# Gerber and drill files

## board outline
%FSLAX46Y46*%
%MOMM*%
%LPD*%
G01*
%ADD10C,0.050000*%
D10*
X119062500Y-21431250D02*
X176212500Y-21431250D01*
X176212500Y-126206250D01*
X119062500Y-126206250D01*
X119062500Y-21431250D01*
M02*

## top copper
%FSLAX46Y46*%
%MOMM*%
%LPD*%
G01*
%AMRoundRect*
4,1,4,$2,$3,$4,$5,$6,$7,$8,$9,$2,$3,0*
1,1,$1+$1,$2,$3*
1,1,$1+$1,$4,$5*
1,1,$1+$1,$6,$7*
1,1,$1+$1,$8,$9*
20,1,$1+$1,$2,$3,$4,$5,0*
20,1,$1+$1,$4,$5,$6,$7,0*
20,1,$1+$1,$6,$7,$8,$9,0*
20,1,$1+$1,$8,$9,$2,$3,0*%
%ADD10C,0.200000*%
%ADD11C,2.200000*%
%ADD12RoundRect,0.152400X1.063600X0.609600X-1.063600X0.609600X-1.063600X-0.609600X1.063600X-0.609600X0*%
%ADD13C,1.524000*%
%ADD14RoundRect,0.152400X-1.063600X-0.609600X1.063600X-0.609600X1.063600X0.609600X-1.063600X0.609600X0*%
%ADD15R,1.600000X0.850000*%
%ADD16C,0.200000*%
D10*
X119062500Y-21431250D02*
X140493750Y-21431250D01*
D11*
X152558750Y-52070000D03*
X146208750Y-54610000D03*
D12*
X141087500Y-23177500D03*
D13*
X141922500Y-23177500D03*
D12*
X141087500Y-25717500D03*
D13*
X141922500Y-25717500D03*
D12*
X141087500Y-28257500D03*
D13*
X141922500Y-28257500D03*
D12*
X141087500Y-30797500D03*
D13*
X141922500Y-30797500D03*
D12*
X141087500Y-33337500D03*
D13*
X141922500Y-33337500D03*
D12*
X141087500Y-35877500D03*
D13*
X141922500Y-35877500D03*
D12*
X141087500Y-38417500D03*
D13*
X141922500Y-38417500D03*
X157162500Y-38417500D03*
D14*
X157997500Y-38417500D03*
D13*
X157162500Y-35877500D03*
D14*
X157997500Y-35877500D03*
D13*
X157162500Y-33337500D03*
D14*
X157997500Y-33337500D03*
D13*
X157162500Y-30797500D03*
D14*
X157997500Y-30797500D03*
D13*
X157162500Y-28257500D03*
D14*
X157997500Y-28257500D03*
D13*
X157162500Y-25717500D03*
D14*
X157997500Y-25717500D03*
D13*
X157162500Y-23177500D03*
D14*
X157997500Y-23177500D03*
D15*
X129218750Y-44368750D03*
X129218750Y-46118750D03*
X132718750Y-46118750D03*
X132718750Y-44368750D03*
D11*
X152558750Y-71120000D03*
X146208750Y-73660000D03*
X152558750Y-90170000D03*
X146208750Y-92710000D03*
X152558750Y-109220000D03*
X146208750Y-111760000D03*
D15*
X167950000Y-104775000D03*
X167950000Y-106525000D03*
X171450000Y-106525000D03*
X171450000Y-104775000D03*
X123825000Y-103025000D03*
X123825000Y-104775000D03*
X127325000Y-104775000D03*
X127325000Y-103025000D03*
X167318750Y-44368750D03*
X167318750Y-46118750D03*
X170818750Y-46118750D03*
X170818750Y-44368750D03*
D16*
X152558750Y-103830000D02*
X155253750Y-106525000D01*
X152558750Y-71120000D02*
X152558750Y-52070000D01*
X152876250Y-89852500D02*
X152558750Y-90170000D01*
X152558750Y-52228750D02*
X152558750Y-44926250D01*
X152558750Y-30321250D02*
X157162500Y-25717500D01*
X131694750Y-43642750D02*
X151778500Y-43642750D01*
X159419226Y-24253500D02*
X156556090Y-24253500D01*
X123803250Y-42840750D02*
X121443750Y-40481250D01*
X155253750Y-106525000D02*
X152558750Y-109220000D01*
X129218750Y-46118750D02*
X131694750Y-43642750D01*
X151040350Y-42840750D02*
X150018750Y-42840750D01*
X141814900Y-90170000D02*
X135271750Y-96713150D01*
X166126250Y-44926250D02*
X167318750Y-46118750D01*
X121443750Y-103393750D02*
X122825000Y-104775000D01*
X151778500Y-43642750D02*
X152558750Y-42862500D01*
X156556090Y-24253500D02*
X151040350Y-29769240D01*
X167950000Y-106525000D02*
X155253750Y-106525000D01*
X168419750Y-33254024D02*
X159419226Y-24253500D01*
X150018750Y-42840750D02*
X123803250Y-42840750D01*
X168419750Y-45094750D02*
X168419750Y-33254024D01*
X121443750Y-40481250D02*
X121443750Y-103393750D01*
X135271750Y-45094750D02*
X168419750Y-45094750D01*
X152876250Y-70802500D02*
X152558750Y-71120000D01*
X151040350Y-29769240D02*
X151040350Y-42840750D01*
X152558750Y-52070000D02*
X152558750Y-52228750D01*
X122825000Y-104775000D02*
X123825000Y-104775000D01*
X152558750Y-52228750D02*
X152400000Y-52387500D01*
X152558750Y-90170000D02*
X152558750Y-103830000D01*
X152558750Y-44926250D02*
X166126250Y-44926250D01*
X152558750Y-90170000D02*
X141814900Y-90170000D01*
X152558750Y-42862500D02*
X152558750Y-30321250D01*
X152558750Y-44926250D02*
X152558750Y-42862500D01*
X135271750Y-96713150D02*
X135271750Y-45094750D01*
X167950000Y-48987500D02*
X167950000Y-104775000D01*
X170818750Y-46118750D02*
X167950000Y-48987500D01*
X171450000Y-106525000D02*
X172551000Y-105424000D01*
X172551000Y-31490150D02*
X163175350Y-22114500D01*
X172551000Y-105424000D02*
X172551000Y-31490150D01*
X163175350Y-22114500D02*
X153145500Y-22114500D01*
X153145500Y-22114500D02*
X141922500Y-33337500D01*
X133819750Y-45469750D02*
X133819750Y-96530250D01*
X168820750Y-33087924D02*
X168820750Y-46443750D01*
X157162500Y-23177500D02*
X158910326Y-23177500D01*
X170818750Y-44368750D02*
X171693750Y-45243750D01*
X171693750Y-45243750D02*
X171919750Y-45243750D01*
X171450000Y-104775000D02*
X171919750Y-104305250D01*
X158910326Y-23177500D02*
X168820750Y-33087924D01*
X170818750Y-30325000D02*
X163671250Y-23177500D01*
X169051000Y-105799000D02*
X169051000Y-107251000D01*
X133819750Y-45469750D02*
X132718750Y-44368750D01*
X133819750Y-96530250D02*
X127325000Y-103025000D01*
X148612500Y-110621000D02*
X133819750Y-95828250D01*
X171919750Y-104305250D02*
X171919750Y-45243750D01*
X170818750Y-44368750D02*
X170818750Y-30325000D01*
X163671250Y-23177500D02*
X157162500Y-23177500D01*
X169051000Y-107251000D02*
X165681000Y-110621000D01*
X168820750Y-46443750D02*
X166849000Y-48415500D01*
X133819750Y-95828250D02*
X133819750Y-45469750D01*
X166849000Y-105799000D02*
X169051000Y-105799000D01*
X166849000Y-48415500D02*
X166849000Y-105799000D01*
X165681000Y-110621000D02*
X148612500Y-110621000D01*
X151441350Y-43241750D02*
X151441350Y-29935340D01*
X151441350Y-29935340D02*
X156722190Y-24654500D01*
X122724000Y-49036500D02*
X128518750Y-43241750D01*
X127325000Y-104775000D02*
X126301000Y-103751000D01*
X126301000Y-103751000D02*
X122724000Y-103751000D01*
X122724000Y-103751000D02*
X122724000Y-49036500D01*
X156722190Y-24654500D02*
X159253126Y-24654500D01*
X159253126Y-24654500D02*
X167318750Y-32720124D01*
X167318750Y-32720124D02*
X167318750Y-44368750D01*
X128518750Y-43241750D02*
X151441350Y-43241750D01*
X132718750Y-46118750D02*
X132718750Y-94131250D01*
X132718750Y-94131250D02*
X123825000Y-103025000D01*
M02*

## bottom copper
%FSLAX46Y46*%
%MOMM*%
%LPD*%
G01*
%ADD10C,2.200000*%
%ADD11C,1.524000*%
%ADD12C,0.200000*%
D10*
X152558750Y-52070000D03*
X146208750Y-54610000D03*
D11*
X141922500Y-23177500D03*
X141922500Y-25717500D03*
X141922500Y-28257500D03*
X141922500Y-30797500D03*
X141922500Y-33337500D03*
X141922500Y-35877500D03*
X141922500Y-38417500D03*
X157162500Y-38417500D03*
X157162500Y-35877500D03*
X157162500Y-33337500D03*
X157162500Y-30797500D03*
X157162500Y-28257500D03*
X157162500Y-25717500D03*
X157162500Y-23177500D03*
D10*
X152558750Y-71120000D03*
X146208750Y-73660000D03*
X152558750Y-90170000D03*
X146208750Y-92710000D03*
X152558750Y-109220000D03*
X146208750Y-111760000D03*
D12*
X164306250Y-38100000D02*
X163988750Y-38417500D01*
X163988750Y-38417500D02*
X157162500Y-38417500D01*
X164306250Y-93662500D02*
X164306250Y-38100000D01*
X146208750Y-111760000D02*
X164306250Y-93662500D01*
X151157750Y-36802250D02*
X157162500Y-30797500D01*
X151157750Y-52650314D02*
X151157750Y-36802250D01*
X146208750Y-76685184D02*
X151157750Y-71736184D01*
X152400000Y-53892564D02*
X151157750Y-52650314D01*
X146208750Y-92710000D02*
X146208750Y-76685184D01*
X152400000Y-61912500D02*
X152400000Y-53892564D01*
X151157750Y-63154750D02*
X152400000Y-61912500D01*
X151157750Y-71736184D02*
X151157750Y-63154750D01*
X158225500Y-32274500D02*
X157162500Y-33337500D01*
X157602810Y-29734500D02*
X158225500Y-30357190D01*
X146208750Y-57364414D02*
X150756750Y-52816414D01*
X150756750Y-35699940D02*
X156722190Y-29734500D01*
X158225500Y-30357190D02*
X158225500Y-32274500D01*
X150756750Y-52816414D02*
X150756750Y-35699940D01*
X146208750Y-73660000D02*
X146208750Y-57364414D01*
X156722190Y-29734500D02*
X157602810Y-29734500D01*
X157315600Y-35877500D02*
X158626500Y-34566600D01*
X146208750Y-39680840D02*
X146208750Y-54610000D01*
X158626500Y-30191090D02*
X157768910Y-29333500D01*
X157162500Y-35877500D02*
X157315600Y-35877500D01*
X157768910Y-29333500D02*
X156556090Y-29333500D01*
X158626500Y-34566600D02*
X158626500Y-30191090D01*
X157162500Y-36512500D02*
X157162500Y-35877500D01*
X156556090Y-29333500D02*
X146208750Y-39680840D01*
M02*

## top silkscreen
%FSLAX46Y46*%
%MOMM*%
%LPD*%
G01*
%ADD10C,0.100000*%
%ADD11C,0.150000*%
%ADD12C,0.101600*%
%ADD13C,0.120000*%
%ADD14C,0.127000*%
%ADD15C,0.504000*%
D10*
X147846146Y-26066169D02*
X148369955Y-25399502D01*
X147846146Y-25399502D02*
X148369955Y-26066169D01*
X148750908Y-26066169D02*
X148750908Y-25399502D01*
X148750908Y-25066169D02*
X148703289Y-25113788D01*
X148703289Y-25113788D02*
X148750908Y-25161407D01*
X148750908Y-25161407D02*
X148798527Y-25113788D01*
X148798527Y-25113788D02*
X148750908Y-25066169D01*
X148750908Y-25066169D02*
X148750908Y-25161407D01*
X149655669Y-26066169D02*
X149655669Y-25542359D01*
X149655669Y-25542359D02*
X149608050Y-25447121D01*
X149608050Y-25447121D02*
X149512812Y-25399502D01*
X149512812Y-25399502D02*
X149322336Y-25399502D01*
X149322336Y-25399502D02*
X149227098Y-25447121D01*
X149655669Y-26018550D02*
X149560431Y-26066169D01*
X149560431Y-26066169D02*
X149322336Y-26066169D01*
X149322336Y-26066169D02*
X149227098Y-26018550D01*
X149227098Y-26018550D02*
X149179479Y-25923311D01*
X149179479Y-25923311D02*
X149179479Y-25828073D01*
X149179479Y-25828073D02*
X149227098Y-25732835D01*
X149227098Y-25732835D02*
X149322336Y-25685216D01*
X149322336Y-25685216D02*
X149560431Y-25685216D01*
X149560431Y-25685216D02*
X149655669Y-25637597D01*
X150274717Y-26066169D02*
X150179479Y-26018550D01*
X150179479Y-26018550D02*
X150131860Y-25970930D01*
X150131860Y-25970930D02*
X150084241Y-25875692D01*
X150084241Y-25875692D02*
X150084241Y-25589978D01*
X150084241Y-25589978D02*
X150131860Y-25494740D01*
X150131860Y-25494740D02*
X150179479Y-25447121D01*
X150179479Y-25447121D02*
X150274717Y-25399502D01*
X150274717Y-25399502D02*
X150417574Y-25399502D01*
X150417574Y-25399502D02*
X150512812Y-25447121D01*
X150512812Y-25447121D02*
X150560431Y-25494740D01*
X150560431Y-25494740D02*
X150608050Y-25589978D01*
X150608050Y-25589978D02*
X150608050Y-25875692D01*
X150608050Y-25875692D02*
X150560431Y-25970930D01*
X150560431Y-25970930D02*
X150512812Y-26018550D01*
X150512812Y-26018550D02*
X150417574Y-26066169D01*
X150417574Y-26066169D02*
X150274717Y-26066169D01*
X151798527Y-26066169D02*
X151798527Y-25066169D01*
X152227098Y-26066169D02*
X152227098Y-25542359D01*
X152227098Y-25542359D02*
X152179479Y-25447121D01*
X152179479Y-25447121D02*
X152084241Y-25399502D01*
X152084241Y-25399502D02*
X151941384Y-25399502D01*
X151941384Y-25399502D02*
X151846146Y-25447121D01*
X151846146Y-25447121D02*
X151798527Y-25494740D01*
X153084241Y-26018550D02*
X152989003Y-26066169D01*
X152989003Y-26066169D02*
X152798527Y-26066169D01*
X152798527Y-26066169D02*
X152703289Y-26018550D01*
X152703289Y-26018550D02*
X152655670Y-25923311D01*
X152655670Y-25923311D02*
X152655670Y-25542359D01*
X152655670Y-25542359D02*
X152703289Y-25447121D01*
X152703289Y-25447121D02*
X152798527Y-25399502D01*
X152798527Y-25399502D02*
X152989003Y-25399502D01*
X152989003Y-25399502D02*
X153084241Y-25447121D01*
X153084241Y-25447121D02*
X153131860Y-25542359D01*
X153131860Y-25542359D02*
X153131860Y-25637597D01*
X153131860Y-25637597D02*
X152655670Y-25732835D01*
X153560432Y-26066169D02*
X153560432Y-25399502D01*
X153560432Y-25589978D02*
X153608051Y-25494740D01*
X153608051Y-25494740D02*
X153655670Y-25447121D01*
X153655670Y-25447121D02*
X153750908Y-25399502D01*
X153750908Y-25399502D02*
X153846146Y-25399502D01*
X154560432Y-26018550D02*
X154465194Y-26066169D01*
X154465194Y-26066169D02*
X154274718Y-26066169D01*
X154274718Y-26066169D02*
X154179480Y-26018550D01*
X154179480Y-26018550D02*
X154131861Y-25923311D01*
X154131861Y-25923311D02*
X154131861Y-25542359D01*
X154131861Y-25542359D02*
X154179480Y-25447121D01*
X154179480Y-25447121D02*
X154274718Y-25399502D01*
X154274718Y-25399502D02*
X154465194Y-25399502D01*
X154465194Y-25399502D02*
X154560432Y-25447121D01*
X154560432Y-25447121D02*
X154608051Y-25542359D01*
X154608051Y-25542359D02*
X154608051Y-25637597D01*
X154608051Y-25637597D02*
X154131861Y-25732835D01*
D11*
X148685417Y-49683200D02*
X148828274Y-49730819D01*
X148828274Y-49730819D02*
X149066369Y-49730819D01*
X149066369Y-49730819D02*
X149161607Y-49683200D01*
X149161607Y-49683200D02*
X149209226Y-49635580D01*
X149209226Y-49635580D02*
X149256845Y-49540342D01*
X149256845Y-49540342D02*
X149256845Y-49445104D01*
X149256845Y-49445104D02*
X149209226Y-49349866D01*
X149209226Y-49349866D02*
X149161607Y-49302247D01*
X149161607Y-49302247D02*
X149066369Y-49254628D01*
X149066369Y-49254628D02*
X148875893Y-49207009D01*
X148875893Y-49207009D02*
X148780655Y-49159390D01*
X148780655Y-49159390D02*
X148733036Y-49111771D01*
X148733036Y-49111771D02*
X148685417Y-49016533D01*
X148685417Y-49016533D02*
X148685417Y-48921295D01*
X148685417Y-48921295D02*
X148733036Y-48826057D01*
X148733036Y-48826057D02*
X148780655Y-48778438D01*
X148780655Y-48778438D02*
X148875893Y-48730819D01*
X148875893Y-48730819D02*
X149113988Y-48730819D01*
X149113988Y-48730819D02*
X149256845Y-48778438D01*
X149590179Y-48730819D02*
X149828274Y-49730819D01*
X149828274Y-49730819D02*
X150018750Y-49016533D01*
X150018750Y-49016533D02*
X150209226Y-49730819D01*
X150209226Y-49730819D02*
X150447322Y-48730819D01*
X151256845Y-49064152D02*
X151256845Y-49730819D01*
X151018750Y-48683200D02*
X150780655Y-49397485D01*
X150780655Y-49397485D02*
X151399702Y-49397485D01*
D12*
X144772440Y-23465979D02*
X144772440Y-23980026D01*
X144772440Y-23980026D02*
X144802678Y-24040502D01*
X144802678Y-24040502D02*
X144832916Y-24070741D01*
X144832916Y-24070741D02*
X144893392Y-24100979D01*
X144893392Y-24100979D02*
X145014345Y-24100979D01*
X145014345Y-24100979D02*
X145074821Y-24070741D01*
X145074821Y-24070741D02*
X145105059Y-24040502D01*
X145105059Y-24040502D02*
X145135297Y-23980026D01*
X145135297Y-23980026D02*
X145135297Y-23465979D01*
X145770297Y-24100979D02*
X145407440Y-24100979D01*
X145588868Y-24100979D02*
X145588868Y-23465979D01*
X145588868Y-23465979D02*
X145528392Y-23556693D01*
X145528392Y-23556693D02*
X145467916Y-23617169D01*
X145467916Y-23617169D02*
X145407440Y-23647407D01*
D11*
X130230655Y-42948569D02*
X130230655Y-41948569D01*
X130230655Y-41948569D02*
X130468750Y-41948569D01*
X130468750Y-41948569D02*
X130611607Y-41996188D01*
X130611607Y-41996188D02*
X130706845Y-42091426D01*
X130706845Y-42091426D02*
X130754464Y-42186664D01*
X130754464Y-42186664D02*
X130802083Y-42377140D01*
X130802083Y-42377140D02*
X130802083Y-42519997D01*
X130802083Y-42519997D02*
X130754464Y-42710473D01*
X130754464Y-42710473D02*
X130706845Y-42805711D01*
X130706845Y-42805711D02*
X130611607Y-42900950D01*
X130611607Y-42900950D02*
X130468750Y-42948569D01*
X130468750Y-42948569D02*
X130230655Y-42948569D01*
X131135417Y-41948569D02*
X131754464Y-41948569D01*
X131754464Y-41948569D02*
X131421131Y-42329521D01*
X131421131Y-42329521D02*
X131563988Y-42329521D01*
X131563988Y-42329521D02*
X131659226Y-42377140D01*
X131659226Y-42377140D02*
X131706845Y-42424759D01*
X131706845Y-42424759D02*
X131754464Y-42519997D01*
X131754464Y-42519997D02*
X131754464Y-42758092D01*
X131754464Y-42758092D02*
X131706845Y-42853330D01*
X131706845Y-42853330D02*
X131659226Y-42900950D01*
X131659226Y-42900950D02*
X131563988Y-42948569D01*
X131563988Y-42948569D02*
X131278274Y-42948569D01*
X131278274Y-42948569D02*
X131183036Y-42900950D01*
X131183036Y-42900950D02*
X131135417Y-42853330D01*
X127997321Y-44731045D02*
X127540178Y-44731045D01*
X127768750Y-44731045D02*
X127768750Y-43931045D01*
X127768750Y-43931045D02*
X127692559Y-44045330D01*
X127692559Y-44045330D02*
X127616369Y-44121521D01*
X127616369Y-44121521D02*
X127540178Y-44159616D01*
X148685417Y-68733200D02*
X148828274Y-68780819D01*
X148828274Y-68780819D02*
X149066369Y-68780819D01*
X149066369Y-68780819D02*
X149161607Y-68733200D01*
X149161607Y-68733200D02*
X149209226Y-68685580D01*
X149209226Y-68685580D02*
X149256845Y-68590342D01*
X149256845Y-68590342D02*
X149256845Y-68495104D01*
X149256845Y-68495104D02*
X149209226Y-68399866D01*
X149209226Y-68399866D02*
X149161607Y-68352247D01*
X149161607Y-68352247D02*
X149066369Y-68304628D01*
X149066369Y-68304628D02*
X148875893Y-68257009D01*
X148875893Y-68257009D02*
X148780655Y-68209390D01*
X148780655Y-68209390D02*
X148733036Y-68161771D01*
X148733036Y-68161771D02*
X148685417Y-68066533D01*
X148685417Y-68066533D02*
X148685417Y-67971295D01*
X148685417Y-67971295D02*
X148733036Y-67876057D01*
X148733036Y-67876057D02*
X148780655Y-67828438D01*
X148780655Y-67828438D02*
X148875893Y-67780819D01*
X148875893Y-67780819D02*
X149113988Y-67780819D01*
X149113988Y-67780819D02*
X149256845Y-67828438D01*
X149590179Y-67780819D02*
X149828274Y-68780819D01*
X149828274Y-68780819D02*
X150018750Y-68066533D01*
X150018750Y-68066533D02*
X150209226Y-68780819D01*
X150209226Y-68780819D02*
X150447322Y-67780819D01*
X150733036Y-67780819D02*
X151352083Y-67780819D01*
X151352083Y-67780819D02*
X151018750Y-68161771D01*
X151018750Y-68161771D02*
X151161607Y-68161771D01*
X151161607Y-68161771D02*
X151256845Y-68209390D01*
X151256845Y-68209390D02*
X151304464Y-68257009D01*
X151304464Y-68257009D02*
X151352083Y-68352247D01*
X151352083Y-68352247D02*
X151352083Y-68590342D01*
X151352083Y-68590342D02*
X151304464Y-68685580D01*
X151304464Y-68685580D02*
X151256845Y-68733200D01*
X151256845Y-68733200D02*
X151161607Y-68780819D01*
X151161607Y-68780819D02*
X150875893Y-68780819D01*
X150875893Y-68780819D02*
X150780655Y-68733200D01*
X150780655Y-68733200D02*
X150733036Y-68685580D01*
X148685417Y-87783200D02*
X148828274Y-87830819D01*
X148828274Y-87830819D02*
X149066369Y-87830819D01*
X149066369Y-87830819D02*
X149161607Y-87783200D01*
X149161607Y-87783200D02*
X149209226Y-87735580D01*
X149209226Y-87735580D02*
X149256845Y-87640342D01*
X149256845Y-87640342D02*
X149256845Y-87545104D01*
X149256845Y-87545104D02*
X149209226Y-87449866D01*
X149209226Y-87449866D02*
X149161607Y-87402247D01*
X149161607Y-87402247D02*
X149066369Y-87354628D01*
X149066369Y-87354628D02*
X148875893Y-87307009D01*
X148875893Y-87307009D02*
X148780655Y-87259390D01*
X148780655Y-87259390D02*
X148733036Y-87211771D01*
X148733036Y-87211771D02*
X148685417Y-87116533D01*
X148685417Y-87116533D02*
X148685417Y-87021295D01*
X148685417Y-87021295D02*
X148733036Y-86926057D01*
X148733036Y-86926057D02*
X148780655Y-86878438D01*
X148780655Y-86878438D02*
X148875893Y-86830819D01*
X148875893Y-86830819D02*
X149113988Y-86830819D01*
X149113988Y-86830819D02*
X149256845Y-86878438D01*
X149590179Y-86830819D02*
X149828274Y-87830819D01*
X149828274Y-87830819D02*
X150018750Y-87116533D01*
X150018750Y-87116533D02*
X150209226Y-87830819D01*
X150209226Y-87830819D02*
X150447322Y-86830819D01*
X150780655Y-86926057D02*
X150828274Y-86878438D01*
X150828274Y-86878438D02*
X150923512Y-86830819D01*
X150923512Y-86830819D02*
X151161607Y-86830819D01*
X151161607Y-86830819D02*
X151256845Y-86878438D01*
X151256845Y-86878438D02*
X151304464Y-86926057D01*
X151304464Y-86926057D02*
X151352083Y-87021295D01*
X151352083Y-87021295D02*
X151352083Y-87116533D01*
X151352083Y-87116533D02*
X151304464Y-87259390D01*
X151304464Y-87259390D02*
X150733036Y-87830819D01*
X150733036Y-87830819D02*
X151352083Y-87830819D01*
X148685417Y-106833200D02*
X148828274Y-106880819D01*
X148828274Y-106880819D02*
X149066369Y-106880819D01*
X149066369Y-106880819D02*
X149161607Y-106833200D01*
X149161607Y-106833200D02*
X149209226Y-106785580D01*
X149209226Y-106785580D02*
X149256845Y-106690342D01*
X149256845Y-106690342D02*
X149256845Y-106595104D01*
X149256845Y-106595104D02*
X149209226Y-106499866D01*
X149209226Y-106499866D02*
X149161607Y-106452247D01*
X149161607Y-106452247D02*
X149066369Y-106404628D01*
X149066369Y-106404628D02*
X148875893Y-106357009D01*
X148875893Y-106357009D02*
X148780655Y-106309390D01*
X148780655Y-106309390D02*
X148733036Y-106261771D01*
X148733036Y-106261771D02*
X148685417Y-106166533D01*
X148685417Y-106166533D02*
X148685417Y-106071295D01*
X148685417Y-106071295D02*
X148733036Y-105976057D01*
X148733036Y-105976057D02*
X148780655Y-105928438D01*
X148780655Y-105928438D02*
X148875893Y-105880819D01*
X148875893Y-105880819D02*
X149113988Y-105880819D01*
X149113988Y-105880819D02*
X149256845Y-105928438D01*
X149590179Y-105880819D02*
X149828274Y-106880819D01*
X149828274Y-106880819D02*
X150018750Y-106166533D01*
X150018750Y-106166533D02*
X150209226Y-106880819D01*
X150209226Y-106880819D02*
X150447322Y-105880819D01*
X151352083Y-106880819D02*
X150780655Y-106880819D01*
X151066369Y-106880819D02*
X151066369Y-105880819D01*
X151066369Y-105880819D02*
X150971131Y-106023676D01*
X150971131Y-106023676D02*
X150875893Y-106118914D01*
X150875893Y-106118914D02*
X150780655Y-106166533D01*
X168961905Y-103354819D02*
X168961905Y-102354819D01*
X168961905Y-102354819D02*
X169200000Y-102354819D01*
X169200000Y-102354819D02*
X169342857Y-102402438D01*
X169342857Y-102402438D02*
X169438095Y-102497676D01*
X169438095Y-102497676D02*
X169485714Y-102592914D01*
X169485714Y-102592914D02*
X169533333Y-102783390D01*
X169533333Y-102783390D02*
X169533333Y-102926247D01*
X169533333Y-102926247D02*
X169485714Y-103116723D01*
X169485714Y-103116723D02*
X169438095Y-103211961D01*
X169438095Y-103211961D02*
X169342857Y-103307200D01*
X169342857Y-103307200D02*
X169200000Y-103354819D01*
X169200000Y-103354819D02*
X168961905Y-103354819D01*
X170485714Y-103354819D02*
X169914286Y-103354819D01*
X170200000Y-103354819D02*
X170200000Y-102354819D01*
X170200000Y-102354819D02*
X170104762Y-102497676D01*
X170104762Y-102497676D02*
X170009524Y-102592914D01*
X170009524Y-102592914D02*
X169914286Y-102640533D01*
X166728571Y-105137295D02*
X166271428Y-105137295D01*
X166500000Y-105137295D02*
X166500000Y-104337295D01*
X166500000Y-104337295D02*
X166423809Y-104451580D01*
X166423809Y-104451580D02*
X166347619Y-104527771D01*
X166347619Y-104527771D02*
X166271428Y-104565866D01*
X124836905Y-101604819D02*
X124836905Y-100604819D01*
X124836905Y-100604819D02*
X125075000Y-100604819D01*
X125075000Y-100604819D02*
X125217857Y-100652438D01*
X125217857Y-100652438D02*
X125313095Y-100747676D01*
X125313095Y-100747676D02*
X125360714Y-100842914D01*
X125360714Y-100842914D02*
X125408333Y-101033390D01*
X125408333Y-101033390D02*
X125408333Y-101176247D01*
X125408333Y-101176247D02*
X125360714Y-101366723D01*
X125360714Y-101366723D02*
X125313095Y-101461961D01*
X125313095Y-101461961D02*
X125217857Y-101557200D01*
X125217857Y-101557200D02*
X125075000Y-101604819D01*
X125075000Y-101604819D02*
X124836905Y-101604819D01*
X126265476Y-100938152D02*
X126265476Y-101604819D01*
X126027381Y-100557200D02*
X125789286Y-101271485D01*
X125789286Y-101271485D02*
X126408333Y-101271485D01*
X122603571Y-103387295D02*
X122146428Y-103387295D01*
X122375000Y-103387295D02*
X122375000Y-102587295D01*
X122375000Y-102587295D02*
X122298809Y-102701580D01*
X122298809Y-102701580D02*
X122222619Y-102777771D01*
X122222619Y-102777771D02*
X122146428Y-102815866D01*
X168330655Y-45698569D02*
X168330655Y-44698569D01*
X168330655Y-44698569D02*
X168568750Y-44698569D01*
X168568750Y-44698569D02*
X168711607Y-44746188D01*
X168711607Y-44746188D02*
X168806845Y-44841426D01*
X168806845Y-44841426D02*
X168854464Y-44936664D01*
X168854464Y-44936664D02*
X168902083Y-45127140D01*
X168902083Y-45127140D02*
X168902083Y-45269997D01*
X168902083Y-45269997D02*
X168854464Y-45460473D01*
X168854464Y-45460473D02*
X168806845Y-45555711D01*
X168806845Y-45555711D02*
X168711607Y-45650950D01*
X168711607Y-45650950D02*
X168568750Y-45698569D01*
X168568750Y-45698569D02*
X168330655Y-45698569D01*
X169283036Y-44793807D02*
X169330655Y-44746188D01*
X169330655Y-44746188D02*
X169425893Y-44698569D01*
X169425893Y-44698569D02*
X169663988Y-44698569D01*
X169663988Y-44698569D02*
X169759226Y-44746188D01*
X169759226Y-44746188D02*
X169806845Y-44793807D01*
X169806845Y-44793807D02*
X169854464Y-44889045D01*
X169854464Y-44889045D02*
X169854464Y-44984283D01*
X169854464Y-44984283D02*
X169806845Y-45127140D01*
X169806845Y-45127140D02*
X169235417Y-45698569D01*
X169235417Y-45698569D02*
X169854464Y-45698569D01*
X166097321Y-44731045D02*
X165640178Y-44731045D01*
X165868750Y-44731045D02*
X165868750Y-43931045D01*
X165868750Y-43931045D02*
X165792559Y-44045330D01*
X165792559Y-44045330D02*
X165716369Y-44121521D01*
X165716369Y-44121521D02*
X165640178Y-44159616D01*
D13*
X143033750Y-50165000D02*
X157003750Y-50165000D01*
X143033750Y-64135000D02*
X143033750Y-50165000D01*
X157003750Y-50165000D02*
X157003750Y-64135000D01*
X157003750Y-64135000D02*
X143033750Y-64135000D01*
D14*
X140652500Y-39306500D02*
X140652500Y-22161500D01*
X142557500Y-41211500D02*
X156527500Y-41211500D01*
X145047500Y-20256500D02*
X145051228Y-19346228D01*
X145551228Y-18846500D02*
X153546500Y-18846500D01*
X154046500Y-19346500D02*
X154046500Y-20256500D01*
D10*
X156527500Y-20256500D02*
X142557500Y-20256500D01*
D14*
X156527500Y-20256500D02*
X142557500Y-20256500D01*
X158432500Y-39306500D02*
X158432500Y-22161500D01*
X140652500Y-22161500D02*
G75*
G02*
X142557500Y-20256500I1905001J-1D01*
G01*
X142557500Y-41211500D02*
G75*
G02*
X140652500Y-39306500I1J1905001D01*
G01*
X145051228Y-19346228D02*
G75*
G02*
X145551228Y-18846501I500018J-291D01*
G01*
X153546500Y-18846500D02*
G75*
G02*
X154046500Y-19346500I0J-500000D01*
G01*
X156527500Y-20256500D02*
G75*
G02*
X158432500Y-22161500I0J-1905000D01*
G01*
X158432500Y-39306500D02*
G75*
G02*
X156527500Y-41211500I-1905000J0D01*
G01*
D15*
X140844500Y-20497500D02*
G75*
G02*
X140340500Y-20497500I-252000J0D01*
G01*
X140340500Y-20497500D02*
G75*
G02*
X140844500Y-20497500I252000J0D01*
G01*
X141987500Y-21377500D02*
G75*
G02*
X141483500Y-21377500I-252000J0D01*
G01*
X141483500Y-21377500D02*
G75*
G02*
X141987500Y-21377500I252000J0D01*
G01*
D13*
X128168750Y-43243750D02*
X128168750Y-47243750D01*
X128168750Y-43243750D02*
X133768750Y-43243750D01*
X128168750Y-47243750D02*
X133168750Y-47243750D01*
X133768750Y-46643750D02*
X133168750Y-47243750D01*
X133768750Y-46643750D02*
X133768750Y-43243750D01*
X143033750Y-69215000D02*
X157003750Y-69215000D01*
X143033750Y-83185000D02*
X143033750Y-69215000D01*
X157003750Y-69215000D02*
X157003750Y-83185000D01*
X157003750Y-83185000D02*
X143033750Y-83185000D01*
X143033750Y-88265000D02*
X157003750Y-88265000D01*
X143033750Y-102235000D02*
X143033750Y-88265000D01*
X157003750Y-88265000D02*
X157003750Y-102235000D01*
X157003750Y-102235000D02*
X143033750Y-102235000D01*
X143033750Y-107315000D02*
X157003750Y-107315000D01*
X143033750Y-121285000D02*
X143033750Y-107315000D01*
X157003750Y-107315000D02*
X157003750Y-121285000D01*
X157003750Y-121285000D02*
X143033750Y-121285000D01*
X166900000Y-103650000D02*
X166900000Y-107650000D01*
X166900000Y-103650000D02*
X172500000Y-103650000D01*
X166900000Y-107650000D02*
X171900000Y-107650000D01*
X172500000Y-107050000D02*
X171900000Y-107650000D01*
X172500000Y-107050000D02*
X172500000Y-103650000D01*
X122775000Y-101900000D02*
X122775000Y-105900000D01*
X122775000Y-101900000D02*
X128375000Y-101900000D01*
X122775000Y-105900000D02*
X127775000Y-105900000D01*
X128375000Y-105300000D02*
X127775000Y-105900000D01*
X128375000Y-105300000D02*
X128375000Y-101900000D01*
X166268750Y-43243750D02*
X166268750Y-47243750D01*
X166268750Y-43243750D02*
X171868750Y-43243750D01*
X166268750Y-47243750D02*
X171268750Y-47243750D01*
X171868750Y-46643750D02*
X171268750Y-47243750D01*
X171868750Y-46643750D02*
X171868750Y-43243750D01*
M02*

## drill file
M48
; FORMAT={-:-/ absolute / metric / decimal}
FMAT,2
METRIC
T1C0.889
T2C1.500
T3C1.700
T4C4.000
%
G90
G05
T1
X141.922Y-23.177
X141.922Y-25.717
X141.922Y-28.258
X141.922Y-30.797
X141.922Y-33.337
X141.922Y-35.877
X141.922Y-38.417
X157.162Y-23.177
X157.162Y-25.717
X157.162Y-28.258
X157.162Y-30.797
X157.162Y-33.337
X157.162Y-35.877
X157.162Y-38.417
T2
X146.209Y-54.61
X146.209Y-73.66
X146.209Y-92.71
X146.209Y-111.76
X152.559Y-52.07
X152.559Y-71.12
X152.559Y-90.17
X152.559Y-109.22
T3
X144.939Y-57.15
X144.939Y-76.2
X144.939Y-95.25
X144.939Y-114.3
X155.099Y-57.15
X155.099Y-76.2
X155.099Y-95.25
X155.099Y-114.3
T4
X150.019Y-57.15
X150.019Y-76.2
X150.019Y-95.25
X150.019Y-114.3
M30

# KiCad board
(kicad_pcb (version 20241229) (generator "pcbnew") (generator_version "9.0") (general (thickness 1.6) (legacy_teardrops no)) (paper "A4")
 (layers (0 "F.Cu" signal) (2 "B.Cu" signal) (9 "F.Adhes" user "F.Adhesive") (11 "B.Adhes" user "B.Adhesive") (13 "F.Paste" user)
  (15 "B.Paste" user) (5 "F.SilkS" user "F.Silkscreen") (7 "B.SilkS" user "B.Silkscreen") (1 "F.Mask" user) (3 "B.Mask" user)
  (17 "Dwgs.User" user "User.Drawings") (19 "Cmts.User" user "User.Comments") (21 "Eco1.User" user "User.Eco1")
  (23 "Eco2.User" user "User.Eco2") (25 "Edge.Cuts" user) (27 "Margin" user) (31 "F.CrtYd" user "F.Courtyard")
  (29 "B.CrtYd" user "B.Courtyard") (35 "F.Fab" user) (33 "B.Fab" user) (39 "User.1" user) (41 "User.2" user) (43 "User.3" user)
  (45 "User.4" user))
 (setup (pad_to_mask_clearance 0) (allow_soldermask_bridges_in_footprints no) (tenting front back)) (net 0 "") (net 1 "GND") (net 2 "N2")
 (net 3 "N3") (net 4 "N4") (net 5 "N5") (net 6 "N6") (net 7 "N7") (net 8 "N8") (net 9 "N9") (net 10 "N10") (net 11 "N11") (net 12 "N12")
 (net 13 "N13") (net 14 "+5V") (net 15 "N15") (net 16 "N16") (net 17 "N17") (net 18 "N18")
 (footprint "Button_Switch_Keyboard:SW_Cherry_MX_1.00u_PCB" (layer "F.Cu") (at 152.55875 52.07)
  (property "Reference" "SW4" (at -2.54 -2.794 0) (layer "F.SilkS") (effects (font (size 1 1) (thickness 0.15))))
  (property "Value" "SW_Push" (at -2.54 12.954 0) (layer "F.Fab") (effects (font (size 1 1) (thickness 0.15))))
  (fp_line (start -9.525 -1.905) (end 4.445 -1.905) (stroke (width 0.12) (type solid)) (layer "F.SilkS"))
  (fp_line (start -9.525 12.065) (end -9.525 -1.905) (stroke (width 0.12) (type solid)) (layer "F.SilkS"))
  (fp_line (start 4.445 -1.905) (end 4.445 12.065) (stroke (width 0.12) (type solid)) (layer "F.SilkS"))
  (fp_line (start 4.445 12.065) (end -9.525 12.065) (stroke (width 0.12) (type solid)) (layer "F.SilkS"))
  (pad "" np_thru_hole circle (at -7.62 5.08) (size 1.7 1.7) (drill 1.7) (layers "*.Cu" "*.Mask"))
  (pad "" np_thru_hole circle (at -2.54 5.08) (size 4 4) (drill 4) (layers "*.Cu" "*.Mask"))
  (pad "" np_thru_hole circle (at 2.54 5.08) (size 1.7 1.7) (drill 1.7) (layers "*.Cu" "*.Mask"))
  (pad "1" thru_hole circle (at 0 0) (size 2.2 2.2) (drill 1.5) (layers "*.Cu" "*.Mask") (remove_unused_layers no) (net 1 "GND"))
  (pad "2" thru_hole circle (at -6.35 2.54) (size 2.2 2.2) (drill 1.5) (layers "*.Cu" "*.Mask") (remove_unused_layers no) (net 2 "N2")))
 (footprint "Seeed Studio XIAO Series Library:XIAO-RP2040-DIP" (layer "F.Cu") (at 149.5425 30.7975)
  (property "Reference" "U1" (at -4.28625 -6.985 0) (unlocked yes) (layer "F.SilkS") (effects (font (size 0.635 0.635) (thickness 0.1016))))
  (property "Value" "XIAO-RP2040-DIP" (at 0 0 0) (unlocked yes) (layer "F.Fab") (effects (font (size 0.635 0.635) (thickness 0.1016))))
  (fp_line (start -8.89 8.509) (end -8.89 -8.636) (stroke (width 0.127) (type solid)) (layer "F.SilkS"))
  (fp_line (start -6.985 10.414) (end 6.985 10.414) (stroke (width 0.127) (type solid)) (layer "F.SilkS"))
  (fp_line (start -4.495 -10.541) (end -4.491272 -11.451272) (stroke (width 0.127) (type solid)) (layer "F.SilkS"))
  (fp_line (start -3.991272 -11.951) (end 4.004 -11.951) (stroke (width 0.127) (type solid)) (layer "F.SilkS"))
  (fp_line (start 4.504 -11.451) (end 4.504 -10.541) (stroke (width 0.127) (type solid)) (layer "F.SilkS"))
  (fp_line (start 6.985 -10.541) (end -6.985 -10.541) (stroke (width 0.1) (type solid)) (layer "F.SilkS"))
  (fp_line (start 6.985 -10.541) (end -6.985 -10.541) (stroke (width 0.127) (type solid)) (layer "F.SilkS"))
  (fp_line (start 8.89 8.509) (end 8.89 -8.636) (stroke (width 0.127) (type solid)) (layer "F.SilkS"))
  (fp_arc (start -8.89 -8.636) (mid -8.332038 -9.983038) (end -6.985 -10.541) (stroke (width 0.127) (type solid)) (layer "F.SilkS"))
  (fp_arc (start -6.985 10.414) (mid -8.332038 9.856038) (end -8.89 8.509) (stroke (width 0.127) (type solid)) (layer "F.SilkS"))
  (fp_arc (start -4.491272 -11.451272) (mid -4.344728 -11.80464) (end -3.991272 -11.951) (stroke (width 0.127) (type default))
   (layer "F.SilkS"))
  (fp_arc (start 4.004 -11.951) (mid 4.357553 -11.804553) (end 4.504 -11.451) (stroke (width 0.127) (type default)) (layer "F.SilkS"))
  (fp_arc (start 6.985 -10.541) (mid 8.332038 -9.983038) (end 8.89 -8.636) (stroke (width 0.127) (type solid)) (layer "F.SilkS"))
  (fp_arc (start 8.89 8.509) (mid 8.332038 9.856038) (end 6.985 10.414) (stroke (width 0.127) (type solid)) (layer "F.SilkS"))
  (fp_circle (center -8.95 -10.3) (end -8.95 -10.554) (stroke (width 0.5) (type solid)) (fill yes) (layer "F.SilkS"))
  (fp_circle (center -7.807 -9.42) (end -7.807 -9.674) (stroke (width 0.5) (type solid)) (fill yes) (layer "F.SilkS"))
  (pad "1" smd roundrect (at -8.455 -7.62 180) (size 2.432 1.524) (layers "F.Cu" "F.Mask") (roundrect_rratio 0.1) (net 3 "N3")
   (thermal_bridge_angle 45))
  (pad "1" thru_hole circle (at -7.62 -7.62 180) (size 1.524 1.524) (drill 0.889) (layers "*.Cu" "*.Mask") (remove_unused_layers no)
   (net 3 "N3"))
  (pad "2" smd roundrect (at -8.455 -5.08 180) (size 2.432 1.524) (layers "F.Cu" "F.Mask") (roundrect_rratio 0.1) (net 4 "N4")
   (thermal_bridge_angle 45))
  (pad "2" thru_hole circle (at -7.62 -5.08 180) (size 1.524 1.524) (drill 0.889) (layers "*.Cu" "*.Mask") (remove_unused_layers no)
   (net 4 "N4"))
  (pad "3" smd roundrect (at -8.455 -2.54 180) (size 2.432 1.524) (layers "F.Cu" "F.Mask") (roundrect_rratio 0.1) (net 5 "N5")
   (thermal_bridge_angle 45))
  (pad "3" thru_hole circle (at -7.62 -2.54 180) (size 1.524 1.524) (drill 0.889) (layers "*.Cu" "*.Mask") (remove_unused_layers no)
   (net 5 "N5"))
  (pad "4" smd roundrect (at -8.455 0 180) (size 2.432 1.524) (layers "F.Cu" "F.Mask") (roundrect_rratio 0.1) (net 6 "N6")
   (thermal_bridge_angle 45))
  (pad "4" thru_hole circle (at -7.62 0 180) (size 1.524 1.524) (drill 0.889) (layers "*.Cu" "*.Mask") (remove_unused_layers no)
   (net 6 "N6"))
  (pad "5" smd roundrect (at -8.455 2.54 180) (size 2.432 1.524) (layers "F.Cu" "F.Mask") (roundrect_rratio 0.1) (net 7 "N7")
   (thermal_bridge_angle 45))
  (pad "5" thru_hole circle (at -7.62 2.54 180) (size 1.524 1.524) (drill 0.889) (layers "*.Cu" "*.Mask") (remove_unused_layers no)
   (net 7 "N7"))
  (pad "6" smd roundrect (at -8.455 5.08 180) (size 2.432 1.524) (layers "F.Cu" "F.Mask") (roundrect_rratio 0.1) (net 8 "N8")
   (thermal_bridge_angle 45))
  (pad "6" thru_hole circle (at -7.62 5.08 180) (size 1.524 1.524) (drill 0.889) (layers "*.Cu" "*.Mask") (remove_unused_layers no)
   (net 8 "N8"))
  (pad "7" smd roundrect (at -8.455 7.62 180) (size 2.432 1.524) (layers "F.Cu" "F.Mask") (roundrect_rratio 0.1) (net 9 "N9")
   (thermal_bridge_angle 45))
  (pad "7" thru_hole circle (at -7.62 7.62 180) (size 1.524 1.524) (drill 0.889) (layers "*.Cu" "*.Mask") (remove_unused_layers no)
   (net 9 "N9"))
  (pad "8" thru_hole circle (at 7.62 7.62) (size 1.524 1.524) (drill 0.889) (layers "*.Cu" "*.Mask") (remove_unused_layers no)
   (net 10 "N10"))
  (pad "8" smd roundrect (at 8.455 7.62) (size 2.432 1.524) (layers "F.Cu" "F.Mask") (roundrect_rratio 0.1) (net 10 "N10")
   (thermal_bridge_angle 45))
  (pad "9" thru_hole circle (at 7.62 5.08) (size 1.524 1.524) (drill 0.889) (layers "*.Cu" "*.Mask") (remove_unused_layers no) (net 2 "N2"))
  (pad "9" smd roundrect (at 8.455 5.08) (size 2.432 1.524) (layers "F.Cu" "F.Mask") (roundrect_rratio 0.1) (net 2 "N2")
   (thermal_bridge_angle 45))
  (pad "10" thru_hole circle (at 7.62 2.54) (size 1.524 1.524) (drill 0.889) (layers "*.Cu" "*.Mask") (remove_unused_layers no)
   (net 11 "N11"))
  (pad "10" smd roundrect (at 8.455 2.54) (size 2.432 1.524) (layers "F.Cu" "F.Mask") (roundrect_rratio 0.1) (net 11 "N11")
   (thermal_bridge_angle 45))
  (pad "11" thru_hole circle (at 7.62 0) (size 1.524 1.524) (drill 0.889) (layers "*.Cu" "*.Mask") (remove_unused_layers no) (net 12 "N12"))
  (pad "11" smd roundrect (at 8.455 0) (size 2.432 1.524) (layers "F.Cu" "F.Mask") (roundrect_rratio 0.1) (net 12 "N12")
   (thermal_bridge_angle 45))
  (pad "12" thru_hole circle (at 7.62 -2.54) (size 1.524 1.524) (drill 0.889) (layers "*.Cu" "*.Mask") (remove_unused_layers no)
   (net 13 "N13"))
  (pad "12" smd roundrect (at 8.455 -2.54) (size 2.432 1.524) (layers "F.Cu" "F.Mask") (roundrect_rratio 0.1) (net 13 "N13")
   (thermal_bridge_angle 45))
  (pad "13" thru_hole circle (at 7.62 -5.08) (size 1.524 1.524) (drill 0.889) (layers "*.Cu" "*.Mask") (remove_unused_layers no)
   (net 1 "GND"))
  (pad "13" smd roundrect (at 8.455 -5.08) (size 2.432 1.524) (layers "F.Cu" "F.Mask") (roundrect_rratio 0.1) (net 1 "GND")
   (thermal_bridge_angle 45))
  (pad "14" thru_hole circle (at 7.62 -7.62) (size 1.524 1.524) (drill 0.889) (layers "*.Cu" "*.Mask") (remove_unused_layers no)
   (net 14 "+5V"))
  (pad "14" smd roundrect (at 8.455 -7.62) (size 2.432 1.524) (layers "F.Cu" "F.Mask") (roundrect_rratio 0.1) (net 14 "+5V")
   (thermal_bridge_angle 45)))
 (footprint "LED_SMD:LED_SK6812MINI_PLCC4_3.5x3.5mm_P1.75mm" (layer "F.Cu") (at 130.96875 45.24375)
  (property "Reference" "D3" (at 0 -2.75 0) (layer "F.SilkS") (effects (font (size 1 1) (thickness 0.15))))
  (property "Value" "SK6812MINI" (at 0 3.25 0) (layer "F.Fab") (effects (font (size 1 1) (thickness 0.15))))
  (fp_line (start -2.8 -2) (end -2.8 2) (stroke (width 0.12) (type default)) (layer "F.SilkS"))
  (fp_line (start -2.8 -2) (end 2.8 -2) (stroke (width 0.12) (type solid)) (layer "F.SilkS"))
  (fp_line (start -2.8 2) (end 2.2 2) (stroke (width 0.12) (type solid)) (layer "F.SilkS"))
  (fp_line (start 2.8 1.4) (end 2.2 2) (stroke (width 0.12) (type default)) (layer "F.SilkS"))
  (fp_line (start 2.8 1.4) (end 2.8 -2) (stroke (width 0.12) (type solid)) (layer "F.SilkS"))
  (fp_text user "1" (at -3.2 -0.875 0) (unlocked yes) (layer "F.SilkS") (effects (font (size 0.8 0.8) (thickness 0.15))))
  (pad "1" smd rect (at -1.75 -0.875) (size 1.6 0.85) (layers "F.Cu" "F.Mask" "F.Paste") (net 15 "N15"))
  (pad "2" smd rect (at -1.75 0.875) (size 1.6 0.85) (layers "F.Cu" "F.Mask" "F.Paste") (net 1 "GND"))
  (pad "3" smd rect (at 1.75 0.875) (size 1.6 0.85) (layers "F.Cu" "F.Mask" "F.Paste") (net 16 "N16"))
  (pad "4" smd rect (at 1.75 -0.875) (size 1.6 0.85) (layers "F.Cu" "F.Mask" "F.Paste") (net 14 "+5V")))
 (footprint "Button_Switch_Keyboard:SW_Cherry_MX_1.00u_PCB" (layer "F.Cu") (at 152.55875 71.12)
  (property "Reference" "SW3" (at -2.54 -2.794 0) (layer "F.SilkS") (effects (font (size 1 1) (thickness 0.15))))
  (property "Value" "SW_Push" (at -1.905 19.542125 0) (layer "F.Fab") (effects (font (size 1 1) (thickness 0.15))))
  (fp_line (start -9.525 -1.905) (end 4.445 -1.905) (stroke (width 0.12) (type solid)) (layer "F.SilkS"))
  (fp_line (start -9.525 12.065) (end -9.525 -1.905) (stroke (width 0.12) (type solid)) (layer "F.SilkS"))
  (fp_line (start 4.445 -1.905) (end 4.445 12.065) (stroke (width 0.12) (type solid)) (layer "F.SilkS"))
  (fp_line (start 4.445 12.065) (end -9.525 12.065) (stroke (width 0.12) (type solid)) (layer "F.SilkS"))
  (pad "" np_thru_hole circle (at -7.62 5.08) (size 1.7 1.7) (drill 1.7) (layers "*.Cu" "*.Mask"))
  (pad "" np_thru_hole circle (at -2.54 5.08) (size 4 4) (drill 4) (layers "*.Cu" "*.Mask"))
  (pad "" np_thru_hole circle (at 2.54 5.08) (size 1.7 1.7) (drill 1.7) (layers "*.Cu" "*.Mask"))
  (pad "1" thru_hole circle (at 0 0) (size 2.2 2.2) (drill 1.5) (layers "*.Cu" "*.Mask") (remove_unused_layers no) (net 1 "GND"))
  (pad "2" thru_hole circle (at -6.35 2.54) (size 2.2 2.2) (drill 1.5) (layers "*.Cu" "*.Mask") (remove_unused_layers no) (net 11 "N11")))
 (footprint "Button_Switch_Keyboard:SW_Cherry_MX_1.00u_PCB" (layer "F.Cu") (at 152.55875 90.17)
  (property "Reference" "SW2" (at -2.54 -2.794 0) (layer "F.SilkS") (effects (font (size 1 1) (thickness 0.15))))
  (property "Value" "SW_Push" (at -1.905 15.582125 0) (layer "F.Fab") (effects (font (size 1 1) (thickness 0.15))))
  (fp_line (start -9.525 -1.905) (end 4.445 -1.905) (stroke (width 0.12) (type solid)) (layer "F.SilkS"))
  (fp_line (start -9.525 12.065) (end -9.525 -1.905) (stroke (width 0.12) (type solid)) (layer "F.SilkS"))
  (fp_line (start 4.445 -1.905) (end 4.445 12.065) (stroke (width 0.12) (type solid)) (layer "F.SilkS"))
  (fp_line (start 4.445 12.065) (end -9.525 12.065) (stroke (width 0.12) (type solid)) (layer "F.SilkS"))
  (pad "" np_thru_hole circle (at -7.62 5.08) (size 1.7 1.7) (drill 1.7) (layers "*.Cu" "*.Mask"))
  (pad "" np_thru_hole circle (at -2.54 5.08) (size 4 4) (drill 4) (layers "*.Cu" "*.Mask"))
  (pad "" np_thru_hole circle (at 2.54 5.08) (size 1.7 1.7) (drill 1.7) (layers "*.Cu" "*.Mask"))
  (pad "1" thru_hole circle (at 0 0) (size 2.2 2.2) (drill 1.5) (layers "*.Cu" "*.Mask") (remove_unused_layers no) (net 1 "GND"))
  (pad "2" thru_hole circle (at -6.35 2.54) (size 2.2 2.2) (drill 1.5) (layers "*.Cu" "*.Mask") (remove_unused_layers no) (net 12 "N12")))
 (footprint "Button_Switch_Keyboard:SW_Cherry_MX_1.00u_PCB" (layer "F.Cu") (at 152.55875 109.22)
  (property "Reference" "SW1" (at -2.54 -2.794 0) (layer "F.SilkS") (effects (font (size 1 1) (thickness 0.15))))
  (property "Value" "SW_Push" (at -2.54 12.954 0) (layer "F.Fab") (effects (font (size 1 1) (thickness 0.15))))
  (fp_line (start -9.525 -1.905) (end 4.445 -1.905) (stroke (width 0.12) (type solid)) (layer "F.SilkS"))
  (fp_line (start -9.525 12.065) (end -9.525 -1.905) (stroke (width 0.12) (type solid)) (layer "F.SilkS"))
  (fp_line (start 4.445 -1.905) (end 4.445 12.065) (stroke (width 0.12) (type solid)) (layer "F.SilkS"))
  (fp_line (start 4.445 12.065) (end -9.525 12.065) (stroke (width 0.12) (type solid)) (layer "F.SilkS"))
  (pad "" np_thru_hole circle (at -7.62 5.08) (size 1.7 1.7) (drill 1.7) (layers "*.Cu" "*.Mask"))
  (pad "" np_thru_hole circle (at -2.54 5.08) (size 4 4) (drill 4) (layers "*.Cu" "*.Mask"))
  (pad "" np_thru_hole circle (at 2.54 5.08) (size 1.7 1.7) (drill 1.7) (layers "*.Cu" "*.Mask"))
  (pad "1" thru_hole circle (at 0 0) (size 2.2 2.2) (drill 1.5) (layers "*.Cu" "*.Mask") (remove_unused_layers no) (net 1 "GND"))
  (pad "2" thru_hole circle (at -6.35 2.54) (size 2.2 2.2) (drill 1.5) (layers "*.Cu" "*.Mask") (remove_unused_layers no) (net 10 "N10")))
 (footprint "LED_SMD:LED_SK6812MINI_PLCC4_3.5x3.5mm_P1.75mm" (layer "F.Cu") (at 169.7 105.65)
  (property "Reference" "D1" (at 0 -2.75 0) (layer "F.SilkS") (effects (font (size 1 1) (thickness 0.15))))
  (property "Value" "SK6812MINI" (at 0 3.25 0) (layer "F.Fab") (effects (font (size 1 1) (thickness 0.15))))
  (fp_line (start -2.8 -2) (end -2.8 2) (stroke (width 0.12) (type default)) (layer "F.SilkS"))
  (fp_line (start -2.8 -2) (end 2.8 -2) (stroke (width 0.12) (type solid)) (layer "F.SilkS"))
  (fp_line (start -2.8 2) (end 2.2 2) (stroke (width 0.12) (type solid)) (layer "F.SilkS"))
  (fp_line (start 2.8 1.4) (end 2.2 2) (stroke (width 0.12) (type default)) (layer "F.SilkS"))
  (fp_line (start 2.8 1.4) (end 2.8 -2) (stroke (width 0.12) (type solid)) (layer "F.SilkS"))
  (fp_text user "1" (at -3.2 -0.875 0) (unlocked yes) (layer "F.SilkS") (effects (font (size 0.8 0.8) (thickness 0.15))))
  (pad "1" smd rect (at -1.75 -0.875) (size 1.6 0.85) (layers "F.Cu" "F.Mask" "F.Paste") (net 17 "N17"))
  (pad "2" smd rect (at -1.75 0.875) (size 1.6 0.85) (layers "F.Cu" "F.Mask" "F.Paste") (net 1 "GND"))
  (pad "3" smd rect (at 1.75 0.875) (size 1.6 0.85) (layers "F.Cu" "F.Mask" "F.Paste") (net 7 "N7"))
  (pad "4" smd rect (at 1.75 -0.875) (size 1.6 0.85) (layers "F.Cu" "F.Mask" "F.Paste") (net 14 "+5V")))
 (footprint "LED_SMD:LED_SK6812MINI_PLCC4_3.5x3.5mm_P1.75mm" (layer "F.Cu") (at 125.575 103.9)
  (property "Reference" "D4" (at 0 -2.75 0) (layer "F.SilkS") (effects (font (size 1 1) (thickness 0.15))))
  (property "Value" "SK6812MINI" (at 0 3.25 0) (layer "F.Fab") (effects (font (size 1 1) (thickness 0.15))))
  (fp_line (start -2.8 -2) (end -2.8 2) (stroke (width 0.12) (type default)) (layer "F.SilkS"))
  (fp_line (start -2.8 -2) (end 2.8 -2) (stroke (width 0.12) (type solid)) (layer "F.SilkS"))
  (fp_line (start -2.8 2) (end 2.2 2) (stroke (width 0.12) (type solid)) (layer "F.SilkS"))
  (fp_line (start 2.8 1.4) (end 2.2 2) (stroke (width 0.12) (type default)) (layer "F.SilkS"))
  (fp_line (start 2.8 1.4) (end 2.8 -2) (stroke (width 0.12) (type solid)) (layer "F.SilkS"))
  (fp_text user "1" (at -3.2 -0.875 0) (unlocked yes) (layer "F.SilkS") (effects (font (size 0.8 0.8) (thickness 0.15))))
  (pad "1" smd rect (at -1.75 -0.875) (size 1.6 0.85) (layers "F.Cu" "F.Mask" "F.Paste") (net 16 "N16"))
  (pad "2" smd rect (at -1.75 0.875) (size 1.6 0.85) (layers "F.Cu" "F.Mask" "F.Paste") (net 1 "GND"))
  (pad "3" smd rect (at 1.75 0.875) (size 1.6 0.85) (layers "F.Cu" "F.Mask" "F.Paste") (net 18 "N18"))
  (pad "4" smd rect (at 1.75 -0.875) (size 1.6 0.85) (layers "F.Cu" "F.Mask" "F.Paste") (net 14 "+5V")))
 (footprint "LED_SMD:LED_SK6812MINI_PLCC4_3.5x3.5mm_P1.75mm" (layer "F.Cu") (at 169.06875 45.24375)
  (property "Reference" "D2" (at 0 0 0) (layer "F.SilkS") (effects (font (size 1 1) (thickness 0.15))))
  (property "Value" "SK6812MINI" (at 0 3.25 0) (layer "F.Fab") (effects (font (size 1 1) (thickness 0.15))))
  (fp_line (start -2.8 -2) (end -2.8 2) (stroke (width 0.12) (type default)) (layer "F.SilkS"))
  (fp_line (start -2.8 -2) (end 2.8 -2) (stroke (width 0.12) (type solid)) (layer "F.SilkS"))
  (fp_line (start -2.8 2) (end 2.2 2) (stroke (width 0.12) (type solid)) (layer "F.SilkS"))
  (fp_line (start 2.8 1.4) (end 2.2 2) (stroke (width 0.12) (type default)) (layer "F.SilkS"))
  (fp_line (start 2.8 1.4) (end 2.8 -2) (stroke (width 0.12) (type solid)) (layer "F.SilkS"))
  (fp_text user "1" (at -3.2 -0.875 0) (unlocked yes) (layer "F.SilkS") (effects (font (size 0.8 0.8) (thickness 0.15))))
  (pad "1" smd rect (at -1.75 -0.875) (size 1.6 0.85) (layers "F.Cu" "F.Mask" "F.Paste") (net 18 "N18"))
  (pad "2" smd rect (at -1.75 0.875) (size 1.6 0.85) (layers "F.Cu" "F.Mask" "F.Paste") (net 1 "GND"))
  (pad "3" smd rect (at 1.75 0.875) (size 1.6 0.85) (layers "F.Cu" "F.Mask" "F.Paste") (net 17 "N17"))
  (pad "4" smd rect (at 1.75 -0.875) (size 1.6 0.85) (layers "F.Cu" "F.Mask" "F.Paste") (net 14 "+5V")))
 (gr_line (start 119.0625 21.43125) (end 140.49375 21.43125) (stroke (width 0.2) (type default)) (layer "F.Cu"))
 (gr_rect (start 119.0625 21.43125) (end 176.2125 126.20625) (stroke (width 0.05) (type default)) (fill no) (layer "Edge.Cuts"))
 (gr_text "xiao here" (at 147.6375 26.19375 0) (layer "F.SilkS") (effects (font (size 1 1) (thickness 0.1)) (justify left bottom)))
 (segment (start 152.55875 103.83) (end 155.25375 106.525) (width 0.2) (layer "F.Cu") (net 1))
 (segment (start 152.55875 71.12) (end 152.55875 52.07) (width 0.2) (layer "F.Cu") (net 1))
 (segment (start 152.87625 89.8525) (end 152.55875 90.17) (width 0.2) (layer "F.Cu") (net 1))
 (segment (start 152.55875 52.22875) (end 152.55875 44.92625) (width 0.2) (layer "F.Cu") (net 1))
 (segment (start 152.55875 30.32125) (end 157.1625 25.7175) (width 0.2) (layer "F.Cu") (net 1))
 (segment (start 131.69475 43.64275) (end 151.7785 43.64275) (width 0.2) (layer "F.Cu") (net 1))
 (segment (start 159.419226 24.2535) (end 156.55609 24.2535) (width 0.2) (layer "F.Cu") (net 1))
 (segment (start 123.80325 42.84075) (end 121.44375 40.48125) (width 0.2) (layer "F.Cu") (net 1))
 (segment (start 155.25375 106.525) (end 152.55875 109.22) (width 0.2) (layer "F.Cu") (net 1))
 (segment (start 129.21875 46.11875) (end 131.69475 43.64275) (width 0.2) (layer "F.Cu") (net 1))
 (segment (start 151.04035 42.84075) (end 150.01875 42.84075) (width 0.2) (layer "F.Cu") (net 1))
 (segment (start 141.8149 90.17) (end 135.27175 96.71315) (width 0.2) (layer "F.Cu") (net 1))
 (segment (start 166.12625 44.92625) (end 167.31875 46.11875) (width 0.2) (layer "F.Cu") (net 1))
 (segment (start 121.44375 103.39375) (end 122.825 104.775) (width 0.2) (layer "F.Cu") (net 1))
 (segment (start 151.7785 43.64275) (end 152.55875 42.8625) (width 0.2) (layer "F.Cu") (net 1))
 (segment (start 156.55609 24.2535) (end 151.04035 29.76924) (width 0.2) (layer "F.Cu") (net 1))
 (segment (start 167.95 106.525) (end 155.25375 106.525) (width 0.2) (layer "F.Cu") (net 1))
 (segment (start 168.41975 33.254024) (end 159.419226 24.2535) (width 0.2) (layer "F.Cu") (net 1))
 (segment (start 150.01875 42.84075) (end 123.80325 42.84075) (width 0.2) (layer "F.Cu") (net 1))
 (segment (start 168.41975 45.09475) (end 168.41975 33.254024) (width 0.2) (layer "F.Cu") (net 1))
 (segment (start 121.44375 40.48125) (end 121.44375 103.39375) (width 0.2) (layer "F.Cu") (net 1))
 (segment (start 135.27175 45.09475) (end 168.41975 45.09475) (width 0.2) (layer "F.Cu") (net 1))
 (segment (start 152.87625 70.8025) (end 152.55875 71.12) (width 0.2) (layer "F.Cu") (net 1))
 (segment (start 151.04035 29.76924) (end 151.04035 42.84075) (width 0.2) (layer "F.Cu") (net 1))
 (segment (start 152.55875 52.07) (end 152.55875 52.22875) (width 0.2) (layer "F.Cu") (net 1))
 (segment (start 122.825 104.775) (end 123.825 104.775) (width 0.2) (layer "F.Cu") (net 1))
 (segment (start 152.55875 52.22875) (end 152.4 52.3875) (width 0.2) (layer "F.Cu") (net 1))
 (segment (start 152.55875 90.17) (end 152.55875 103.83) (width 0.2) (layer "F.Cu") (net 1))
 (segment (start 152.55875 44.92625) (end 166.12625 44.92625) (width 0.2) (layer "F.Cu") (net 1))
 (segment (start 152.55875 90.17) (end 141.8149 90.17) (width 0.2) (layer "F.Cu") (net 1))
 (segment (start 152.55875 42.8625) (end 152.55875 30.32125) (width 0.2) (layer "F.Cu") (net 1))
 (segment (start 152.55875 44.92625) (end 152.55875 42.8625) (width 0.2) (layer "F.Cu") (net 1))
 (segment (start 135.27175 96.71315) (end 135.27175 45.09475) (width 0.2) (layer "F.Cu") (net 1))
 (segment (start 167.95 48.9875) (end 167.95 104.775) (width 0.2) (layer "F.Cu") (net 17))
 (segment (start 170.81875 46.11875) (end 167.95 48.9875) (width 0.2) (layer "F.Cu") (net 17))
 (segment (start 171.45 106.525) (end 172.551 105.424) (width 0.2) (layer "F.Cu") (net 7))
 (segment (start 172.551 31.49015) (end 163.17535 22.1145) (width 0.2) (layer "F.Cu") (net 7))
 (segment (start 172.551 105.424) (end 172.551 31.49015) (width 0.2) (layer "F.Cu") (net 7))
 (segment (start 163.17535 22.1145) (end 153.1455 22.1145) (width 0.2) (layer "F.Cu") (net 7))
 (segment (start 153.1455 22.1145) (end 141.9225 33.3375) (width 0.2) (layer "F.Cu") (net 7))
 (segment (start 133.81975 45.46975) (end 133.81975 96.53025) (width 0.2) (layer "F.Cu") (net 14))
 (segment (start 168.82075 33.087924) (end 168.82075 46.44375) (width 0.2) (layer "F.Cu") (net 14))
 (segment (start 157.1625 23.1775) (end 158.910326 23.1775) (width 0.2) (layer "F.Cu") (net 14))
 (segment (start 170.81875 44.36875) (end 171.69375 45.24375) (width 0.2) (layer "F.Cu") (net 14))
 (segment (start 171.69375 45.24375) (end 171.91975 45.24375) (width 0.2) (layer "F.Cu") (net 14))
 (segment (start 171.45 104.775) (end 171.91975 104.30525) (width 0.2) (layer "F.Cu") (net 14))
 (segment (start 158.910326 23.1775) (end 168.82075 33.087924) (width 0.2) (layer "F.Cu") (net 14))
 (segment (start 170.81875 30.325) (end 163.67125 23.1775) (width 0.2) (layer "F.Cu") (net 14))
 (segment (start 169.051 105.799) (end 169.051 107.251) (width 0.2) (layer "F.Cu") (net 14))
 (segment (start 133.81975 45.46975) (end 132.71875 44.36875) (width 0.2) (layer "F.Cu") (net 14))
 (segment (start 133.81975 96.53025) (end 127.325 103.025) (width 0.2) (layer "F.Cu") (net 14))
 (segment (start 148.6125 110.621) (end 133.81975 95.82825) (width 0.2) (layer "F.Cu") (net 14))
 (segment (start 171.91975 104.30525) (end 171.91975 45.24375) (width 0.2) (layer "F.Cu") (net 14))
 (segment (start 170.81875 44.36875) (end 170.81875 30.325) (width 0.2) (layer "F.Cu") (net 14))
 (segment (start 163.67125 23.1775) (end 157.1625 23.1775) (width 0.2) (layer "F.Cu") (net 14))
 (segment (start 169.051 107.251) (end 165.681 110.621) (width 0.2) (layer "F.Cu") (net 14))
 (segment (start 168.82075 46.44375) (end 166.849 48.4155) (width 0.2) (layer "F.Cu") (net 14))
 (segment (start 133.81975 95.82825) (end 133.81975 45.46975) (width 0.2) (layer "F.Cu") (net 14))
 (segment (start 166.849 105.799) (end 169.051 105.799) (width 0.2) (layer "F.Cu") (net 14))
 (segment (start 166.849 48.4155) (end 166.849 105.799) (width 0.2) (layer "F.Cu") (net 14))
 (segment (start 165.681 110.621) (end 148.6125 110.621) (width 0.2) (layer "F.Cu") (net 14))
 (segment (start 151.44135 43.24175) (end 151.44135 29.93534) (width 0.2) (layer "F.Cu") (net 18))
 (segment (start 151.44135 29.93534) (end 156.72219 24.6545) (width 0.2) (layer "F.Cu") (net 18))
 (segment (start 122.724 49.0365) (end 128.51875 43.24175) (width 0.2) (layer "F.Cu") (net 18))
 (segment (start 127.325 104.775) (end 126.301 103.751) (width 0.2) (layer "F.Cu") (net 18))
 (segment (start 126.301 103.751) (end 122.724 103.751) (width 0.2) (layer "F.Cu") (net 18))
 (segment (start 122.724 103.751) (end 122.724 49.0365) (width 0.2) (layer "F.Cu") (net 18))
 (segment (start 156.72219 24.6545) (end 159.253126 24.6545) (width 0.2) (layer "F.Cu") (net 18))
 (segment (start 159.253126 24.6545) (end 167.31875 32.720124) (width 0.2) (layer "F.Cu") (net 18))
 (segment (start 167.31875 32.720124) (end 167.31875 44.36875) (width 0.2) (layer "F.Cu") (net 18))
 (segment (start 128.51875 43.24175) (end 151.44135 43.24175) (width 0.2) (layer "F.Cu") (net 18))
 (segment (start 132.71875 46.11875) (end 132.71875 94.13125) (width 0.2) (layer "F.Cu") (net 16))
 (segment (start 132.71875 94.13125) (end 123.825 103.025) (width 0.2) (layer "F.Cu") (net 16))
 (segment (start 164.30625 38.1) (end 163.98875 38.4175) (width 0.2) (layer "B.Cu") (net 10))
 (segment (start 163.98875 38.4175) (end 157.1625 38.4175) (width 0.2) (layer "B.Cu") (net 10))
 (segment (start 164.30625 93.6625) (end 164.30625 38.1) (width 0.2) (layer "B.Cu") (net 10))
 (segment (start 146.20875 111.76) (end 164.30625 93.6625) (width 0.2) (layer "B.Cu") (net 10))
 (segment (start 151.15775 36.80225) (end 157.1625 30.7975) (width 0.2) (layer "B.Cu") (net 12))
 (segment (start 151.15775 52.650314) (end 151.15775 36.80225) (width 0.2) (layer "B.Cu") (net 12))
 (segment (start 146.20875 76.685184) (end 151.15775 71.736184) (width 0.2) (layer "B.Cu") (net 12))
 (segment (start 152.4 53.892564) (end 151.15775 52.650314) (width 0.2) (layer "B.Cu") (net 12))
 (segment (start 146.20875 92.71) (end 146.20875 76.685184) (width 0.2) (layer "B.Cu") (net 12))
 (segment (start 152.4 61.9125) (end 152.4 53.892564) (width 0.2) (layer "B.Cu") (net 12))
 (segment (start 151.15775 63.15475) (end 152.4 61.9125) (width 0.2) (layer "B.Cu") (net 12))
 (segment (start 151.15775 71.736184) (end 151.15775 63.15475) (width 0.2) (layer "B.Cu") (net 12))
 (segment (start 158.2255 32.2745) (end 157.1625 33.3375) (width 0.2) (layer "B.Cu") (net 11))
 (segment (start 157.60281 29.7345) (end 158.2255 30.35719) (width 0.2) (layer "B.Cu") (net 11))
 (segment (start 146.20875 57.364414) (end 150.75675 52.816414) (width 0.2) (layer "B.Cu") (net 11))
 (segment (start 150.75675 35.69994) (end 156.72219 29.7345) (width 0.2) (layer "B.Cu") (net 11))
 (segment (start 158.2255 30.35719) (end 158.2255 32.2745) (width 0.2) (layer "B.Cu") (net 11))
 (segment (start 150.75675 52.816414) (end 150.75675 35.69994) (width 0.2) (layer "B.Cu") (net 11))
 (segment (start 146.20875 73.66) (end 146.20875 57.364414) (width 0.2) (layer "B.Cu") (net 11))
 (segment (start 156.72219 29.7345) (end 157.60281 29.7345) (width 0.2) (layer "B.Cu") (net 11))
 (segment (start 157.3156 35.8775) (end 158.6265 34.5666) (width 0.2) (layer "B.Cu") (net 2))
 (segment (start 146.20875 39.68084) (end 146.20875 54.61) (width 0.2) (layer "B.Cu") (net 2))
 (segment (start 158.6265 30.19109) (end 157.76891 29.3335) (width 0.2) (layer "B.Cu") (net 2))
 (segment (start 157.1625 35.8775) (end 157.3156 35.8775) (width 0.2) (layer "B.Cu") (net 2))
 (segment (start 157.76891 29.3335) (end 156.55609 29.3335) (width 0.2) (layer "B.Cu") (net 2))
 (segment (start 158.6265 34.5666) (end 158.6265 30.19109) (width 0.2) (layer "B.Cu") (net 2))
 (segment (start 157.1625 36.5125) (end 157.1625 35.8775) (width 0.2) (layer "B.Cu") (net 2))
 (segment (start 156.55609 29.3335) (end 146.20875 39.68084) (width 0.2) (layer "B.Cu") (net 2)))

